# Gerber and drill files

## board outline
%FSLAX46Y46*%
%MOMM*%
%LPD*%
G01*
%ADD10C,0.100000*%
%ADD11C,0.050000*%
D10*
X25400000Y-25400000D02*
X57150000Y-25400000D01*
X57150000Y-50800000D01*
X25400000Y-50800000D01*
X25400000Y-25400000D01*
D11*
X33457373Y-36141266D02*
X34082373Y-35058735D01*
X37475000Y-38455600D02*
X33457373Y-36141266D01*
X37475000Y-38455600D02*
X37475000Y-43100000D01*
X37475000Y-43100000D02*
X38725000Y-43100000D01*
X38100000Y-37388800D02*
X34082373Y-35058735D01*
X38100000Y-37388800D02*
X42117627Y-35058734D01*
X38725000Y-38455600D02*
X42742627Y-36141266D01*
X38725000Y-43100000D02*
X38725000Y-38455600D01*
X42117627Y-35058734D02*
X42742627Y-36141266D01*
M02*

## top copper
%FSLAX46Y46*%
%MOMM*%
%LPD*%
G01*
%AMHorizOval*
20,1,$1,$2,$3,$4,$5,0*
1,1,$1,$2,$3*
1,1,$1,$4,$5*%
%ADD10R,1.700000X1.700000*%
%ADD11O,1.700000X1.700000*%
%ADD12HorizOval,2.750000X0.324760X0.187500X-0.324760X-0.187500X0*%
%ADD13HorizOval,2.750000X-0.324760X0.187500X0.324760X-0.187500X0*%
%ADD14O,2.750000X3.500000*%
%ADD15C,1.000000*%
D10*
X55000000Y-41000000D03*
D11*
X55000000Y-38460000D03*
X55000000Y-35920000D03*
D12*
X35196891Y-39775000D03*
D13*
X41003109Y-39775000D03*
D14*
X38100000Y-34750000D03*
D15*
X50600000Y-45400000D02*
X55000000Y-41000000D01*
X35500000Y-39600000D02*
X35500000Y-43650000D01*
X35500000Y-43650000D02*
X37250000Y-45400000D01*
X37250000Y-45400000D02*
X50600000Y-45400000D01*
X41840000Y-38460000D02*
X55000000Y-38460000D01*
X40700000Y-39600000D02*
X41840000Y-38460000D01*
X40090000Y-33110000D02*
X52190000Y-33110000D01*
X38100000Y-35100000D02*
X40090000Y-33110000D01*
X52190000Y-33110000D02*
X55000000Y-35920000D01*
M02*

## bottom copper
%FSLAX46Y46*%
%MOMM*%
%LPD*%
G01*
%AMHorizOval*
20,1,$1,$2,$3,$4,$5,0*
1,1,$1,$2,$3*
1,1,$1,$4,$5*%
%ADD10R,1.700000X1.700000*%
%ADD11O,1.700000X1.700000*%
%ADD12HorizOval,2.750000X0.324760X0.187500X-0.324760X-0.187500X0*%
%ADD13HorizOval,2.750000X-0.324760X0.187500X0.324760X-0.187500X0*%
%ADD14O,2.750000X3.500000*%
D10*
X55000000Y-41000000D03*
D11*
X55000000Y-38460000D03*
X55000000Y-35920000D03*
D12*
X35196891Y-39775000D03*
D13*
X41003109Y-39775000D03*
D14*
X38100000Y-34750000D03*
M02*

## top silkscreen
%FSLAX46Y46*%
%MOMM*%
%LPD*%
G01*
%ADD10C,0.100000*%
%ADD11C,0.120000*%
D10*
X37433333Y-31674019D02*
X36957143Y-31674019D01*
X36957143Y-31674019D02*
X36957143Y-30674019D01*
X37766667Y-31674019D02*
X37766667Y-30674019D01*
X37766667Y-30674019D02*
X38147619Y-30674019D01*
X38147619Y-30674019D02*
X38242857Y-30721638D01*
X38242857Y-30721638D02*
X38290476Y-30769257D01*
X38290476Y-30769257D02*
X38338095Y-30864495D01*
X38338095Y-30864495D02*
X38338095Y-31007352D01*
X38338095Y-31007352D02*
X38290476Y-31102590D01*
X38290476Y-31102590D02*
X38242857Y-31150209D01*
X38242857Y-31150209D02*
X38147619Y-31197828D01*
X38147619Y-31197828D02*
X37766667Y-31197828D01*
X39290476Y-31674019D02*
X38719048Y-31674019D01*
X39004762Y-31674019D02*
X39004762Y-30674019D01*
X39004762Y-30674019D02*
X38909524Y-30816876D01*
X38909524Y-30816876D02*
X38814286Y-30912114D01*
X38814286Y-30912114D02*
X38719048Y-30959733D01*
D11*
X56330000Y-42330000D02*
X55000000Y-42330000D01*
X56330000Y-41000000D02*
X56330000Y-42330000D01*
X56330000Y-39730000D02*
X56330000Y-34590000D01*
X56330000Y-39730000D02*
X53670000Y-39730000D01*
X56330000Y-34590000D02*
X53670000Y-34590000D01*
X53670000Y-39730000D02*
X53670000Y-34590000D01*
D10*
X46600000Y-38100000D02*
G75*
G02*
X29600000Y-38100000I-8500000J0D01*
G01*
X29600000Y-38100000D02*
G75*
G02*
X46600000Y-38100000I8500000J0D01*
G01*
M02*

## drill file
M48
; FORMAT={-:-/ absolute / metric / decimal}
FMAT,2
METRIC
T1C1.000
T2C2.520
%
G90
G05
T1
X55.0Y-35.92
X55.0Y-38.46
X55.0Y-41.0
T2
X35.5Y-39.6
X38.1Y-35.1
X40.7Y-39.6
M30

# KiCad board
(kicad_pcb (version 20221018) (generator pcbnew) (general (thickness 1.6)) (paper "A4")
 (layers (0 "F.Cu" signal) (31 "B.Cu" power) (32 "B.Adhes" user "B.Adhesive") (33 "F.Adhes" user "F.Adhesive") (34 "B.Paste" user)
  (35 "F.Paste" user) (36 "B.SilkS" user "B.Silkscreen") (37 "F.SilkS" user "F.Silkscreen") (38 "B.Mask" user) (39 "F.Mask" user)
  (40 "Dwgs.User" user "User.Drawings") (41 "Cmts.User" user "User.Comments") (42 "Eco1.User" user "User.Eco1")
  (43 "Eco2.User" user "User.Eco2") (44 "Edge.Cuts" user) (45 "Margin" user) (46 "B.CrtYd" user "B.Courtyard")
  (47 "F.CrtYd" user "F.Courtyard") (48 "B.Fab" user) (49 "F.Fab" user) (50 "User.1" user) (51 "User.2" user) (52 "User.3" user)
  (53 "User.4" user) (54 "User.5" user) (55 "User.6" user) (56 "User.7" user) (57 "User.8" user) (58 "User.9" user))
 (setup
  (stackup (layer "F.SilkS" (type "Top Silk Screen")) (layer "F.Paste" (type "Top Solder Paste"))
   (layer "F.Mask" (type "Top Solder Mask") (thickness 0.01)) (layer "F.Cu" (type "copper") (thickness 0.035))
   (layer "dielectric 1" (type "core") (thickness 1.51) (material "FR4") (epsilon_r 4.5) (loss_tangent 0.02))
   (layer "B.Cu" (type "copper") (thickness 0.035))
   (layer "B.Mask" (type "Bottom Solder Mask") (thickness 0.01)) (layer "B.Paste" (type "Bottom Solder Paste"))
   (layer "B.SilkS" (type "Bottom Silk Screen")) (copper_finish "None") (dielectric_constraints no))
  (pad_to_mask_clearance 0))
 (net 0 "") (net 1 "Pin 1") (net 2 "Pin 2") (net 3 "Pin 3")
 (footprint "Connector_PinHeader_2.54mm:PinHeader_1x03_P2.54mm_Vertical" (layer "F.Cu") (at 55 41 180)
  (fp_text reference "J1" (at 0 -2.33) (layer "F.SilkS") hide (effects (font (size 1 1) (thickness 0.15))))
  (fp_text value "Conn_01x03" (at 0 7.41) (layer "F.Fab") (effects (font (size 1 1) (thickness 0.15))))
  (fp_line (start -1.33 -1.33) (end 0 -1.33) (stroke (width 0.12) (type solid)) (layer "F.SilkS"))
  (fp_line (start -1.33 0) (end -1.33 -1.33) (stroke (width 0.12) (type solid)) (layer "F.SilkS"))
  (fp_line (start -1.33 1.27) (end -1.33 6.41) (stroke (width 0.12) (type solid)) (layer "F.SilkS"))
  (fp_line (start -1.33 1.27) (end 1.33 1.27) (stroke (width 0.12) (type solid)) (layer "F.SilkS"))
  (fp_line (start -1.33 6.41) (end 1.33 6.41) (stroke (width 0.12) (type solid)) (layer "F.SilkS"))
  (fp_line (start 1.33 1.27) (end 1.33 6.41) (stroke (width 0.12) (type solid)) (layer "F.SilkS"))
  (pad "1" thru_hole rect (at 0 0 180) (size 1.7 1.7) (drill 1) (layers "*.Cu" "*.Mask") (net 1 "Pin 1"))
  (pad "2" thru_hole oval (at 0 2.54 180) (size 1.7 1.7) (drill 1) (layers "*.Cu" "*.Mask") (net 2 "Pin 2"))
  (pad "3" thru_hole oval (at 0 5.08 180) (size 1.7 1.7) (drill 1) (layers "*.Cu" "*.Mask") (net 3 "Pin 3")))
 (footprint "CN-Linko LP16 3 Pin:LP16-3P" (layer "F.Cu") (at 38.1 38.1)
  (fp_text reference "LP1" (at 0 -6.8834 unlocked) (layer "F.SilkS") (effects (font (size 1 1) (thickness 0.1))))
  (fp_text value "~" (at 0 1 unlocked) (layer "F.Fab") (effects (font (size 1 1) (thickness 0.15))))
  (fp_circle (center 0 0) (end 8.5 0) (stroke (width 0.1) (type default)) (fill none) (layer "F.SilkS"))
  (fp_line (start -4.642627 -1.958734) (end -4.017627 -3.041265) (stroke (width 0.05) (type default)) (layer "Edge.Cuts"))
  (fp_line (start -0.625 0.3556) (end -4.642627 -1.958734) (stroke (width 0.05) (type default)) (layer "Edge.Cuts"))
  (fp_line (start -0.625 0.3556) (end -0.625 5) (stroke (width 0.05) (type default)) (layer "Edge.Cuts"))
  (fp_line (start -0.625 5) (end 0.625 5) (stroke (width 0.05) (type default)) (layer "Edge.Cuts"))
  (fp_line (start 0 -0.7112) (end -4.017627 -3.041265) (stroke (width 0.05) (type default)) (layer "Edge.Cuts"))
  (fp_line (start 0 -0.7112) (end 4.017627 -3.041266) (stroke (width 0.05) (type default)) (layer "Edge.Cuts"))
  (fp_line (start 0.625 0.3556) (end 4.642627 -1.958734) (stroke (width 0.05) (type default)) (layer "Edge.Cuts"))
  (fp_line (start 0.625 5) (end 0.625 0.3556) (stroke (width 0.05) (type default)) (layer "Edge.Cuts"))
  (fp_line (start 4.017627 -3.041266) (end 4.642627 -1.958734) (stroke (width 0.05) (type default)) (layer "Edge.Cuts"))
  (pad "1" thru_hole oval (at -2.6 1.5 120) (size 2.75 3.5) (drill 2.52 (offset 0 -0.35)) (layers "*.Cu" "*.Mask") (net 1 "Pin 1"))
  (pad "2" thru_hole oval (at 2.6 1.5 240) (size 2.75 3.5) (drill 2.52 (offset 0 -0.35)) (layers "*.Cu" "*.Mask") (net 2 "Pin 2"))
  (pad "3" thru_hole oval (at 0 -3) (size 2.75 3.5) (drill 2.52 (offset 0 -0.35)) (layers "*.Cu" "*.Mask") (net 3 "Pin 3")))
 (gr_rect (start 25.4 25.4) (end 57.15 50.8) (stroke (width 0.1) (type default)) (fill none) (layer "Edge.Cuts"))
 (segment (start 50.6 45.4) (end 55 41) (width 1) (layer "F.Cu") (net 1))
 (segment (start 35.5 39.6) (end 35.5 43.65) (width 1) (layer "F.Cu") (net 1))
 (segment (start 35.5 43.65) (end 37.25 45.4) (width 1) (layer "F.Cu") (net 1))
 (segment (start 37.25 45.4) (end 50.6 45.4) (width 1) (layer "F.Cu") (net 1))
 (segment (start 41.84 38.46) (end 55 38.46) (width 1) (layer "F.Cu") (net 2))
 (segment (start 40.7 39.6) (end 41.84 38.46) (width 1) (layer "F.Cu") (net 2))
 (segment (start 40.09 33.11) (end 52.19 33.11) (width 1) (layer "F.Cu") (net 3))
 (segment (start 38.1 35.1) (end 40.09 33.11) (width 1) (layer "F.Cu") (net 3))
 (segment (start 52.19 33.11) (end 55 35.92) (width 1) (layer "F.Cu") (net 3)))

